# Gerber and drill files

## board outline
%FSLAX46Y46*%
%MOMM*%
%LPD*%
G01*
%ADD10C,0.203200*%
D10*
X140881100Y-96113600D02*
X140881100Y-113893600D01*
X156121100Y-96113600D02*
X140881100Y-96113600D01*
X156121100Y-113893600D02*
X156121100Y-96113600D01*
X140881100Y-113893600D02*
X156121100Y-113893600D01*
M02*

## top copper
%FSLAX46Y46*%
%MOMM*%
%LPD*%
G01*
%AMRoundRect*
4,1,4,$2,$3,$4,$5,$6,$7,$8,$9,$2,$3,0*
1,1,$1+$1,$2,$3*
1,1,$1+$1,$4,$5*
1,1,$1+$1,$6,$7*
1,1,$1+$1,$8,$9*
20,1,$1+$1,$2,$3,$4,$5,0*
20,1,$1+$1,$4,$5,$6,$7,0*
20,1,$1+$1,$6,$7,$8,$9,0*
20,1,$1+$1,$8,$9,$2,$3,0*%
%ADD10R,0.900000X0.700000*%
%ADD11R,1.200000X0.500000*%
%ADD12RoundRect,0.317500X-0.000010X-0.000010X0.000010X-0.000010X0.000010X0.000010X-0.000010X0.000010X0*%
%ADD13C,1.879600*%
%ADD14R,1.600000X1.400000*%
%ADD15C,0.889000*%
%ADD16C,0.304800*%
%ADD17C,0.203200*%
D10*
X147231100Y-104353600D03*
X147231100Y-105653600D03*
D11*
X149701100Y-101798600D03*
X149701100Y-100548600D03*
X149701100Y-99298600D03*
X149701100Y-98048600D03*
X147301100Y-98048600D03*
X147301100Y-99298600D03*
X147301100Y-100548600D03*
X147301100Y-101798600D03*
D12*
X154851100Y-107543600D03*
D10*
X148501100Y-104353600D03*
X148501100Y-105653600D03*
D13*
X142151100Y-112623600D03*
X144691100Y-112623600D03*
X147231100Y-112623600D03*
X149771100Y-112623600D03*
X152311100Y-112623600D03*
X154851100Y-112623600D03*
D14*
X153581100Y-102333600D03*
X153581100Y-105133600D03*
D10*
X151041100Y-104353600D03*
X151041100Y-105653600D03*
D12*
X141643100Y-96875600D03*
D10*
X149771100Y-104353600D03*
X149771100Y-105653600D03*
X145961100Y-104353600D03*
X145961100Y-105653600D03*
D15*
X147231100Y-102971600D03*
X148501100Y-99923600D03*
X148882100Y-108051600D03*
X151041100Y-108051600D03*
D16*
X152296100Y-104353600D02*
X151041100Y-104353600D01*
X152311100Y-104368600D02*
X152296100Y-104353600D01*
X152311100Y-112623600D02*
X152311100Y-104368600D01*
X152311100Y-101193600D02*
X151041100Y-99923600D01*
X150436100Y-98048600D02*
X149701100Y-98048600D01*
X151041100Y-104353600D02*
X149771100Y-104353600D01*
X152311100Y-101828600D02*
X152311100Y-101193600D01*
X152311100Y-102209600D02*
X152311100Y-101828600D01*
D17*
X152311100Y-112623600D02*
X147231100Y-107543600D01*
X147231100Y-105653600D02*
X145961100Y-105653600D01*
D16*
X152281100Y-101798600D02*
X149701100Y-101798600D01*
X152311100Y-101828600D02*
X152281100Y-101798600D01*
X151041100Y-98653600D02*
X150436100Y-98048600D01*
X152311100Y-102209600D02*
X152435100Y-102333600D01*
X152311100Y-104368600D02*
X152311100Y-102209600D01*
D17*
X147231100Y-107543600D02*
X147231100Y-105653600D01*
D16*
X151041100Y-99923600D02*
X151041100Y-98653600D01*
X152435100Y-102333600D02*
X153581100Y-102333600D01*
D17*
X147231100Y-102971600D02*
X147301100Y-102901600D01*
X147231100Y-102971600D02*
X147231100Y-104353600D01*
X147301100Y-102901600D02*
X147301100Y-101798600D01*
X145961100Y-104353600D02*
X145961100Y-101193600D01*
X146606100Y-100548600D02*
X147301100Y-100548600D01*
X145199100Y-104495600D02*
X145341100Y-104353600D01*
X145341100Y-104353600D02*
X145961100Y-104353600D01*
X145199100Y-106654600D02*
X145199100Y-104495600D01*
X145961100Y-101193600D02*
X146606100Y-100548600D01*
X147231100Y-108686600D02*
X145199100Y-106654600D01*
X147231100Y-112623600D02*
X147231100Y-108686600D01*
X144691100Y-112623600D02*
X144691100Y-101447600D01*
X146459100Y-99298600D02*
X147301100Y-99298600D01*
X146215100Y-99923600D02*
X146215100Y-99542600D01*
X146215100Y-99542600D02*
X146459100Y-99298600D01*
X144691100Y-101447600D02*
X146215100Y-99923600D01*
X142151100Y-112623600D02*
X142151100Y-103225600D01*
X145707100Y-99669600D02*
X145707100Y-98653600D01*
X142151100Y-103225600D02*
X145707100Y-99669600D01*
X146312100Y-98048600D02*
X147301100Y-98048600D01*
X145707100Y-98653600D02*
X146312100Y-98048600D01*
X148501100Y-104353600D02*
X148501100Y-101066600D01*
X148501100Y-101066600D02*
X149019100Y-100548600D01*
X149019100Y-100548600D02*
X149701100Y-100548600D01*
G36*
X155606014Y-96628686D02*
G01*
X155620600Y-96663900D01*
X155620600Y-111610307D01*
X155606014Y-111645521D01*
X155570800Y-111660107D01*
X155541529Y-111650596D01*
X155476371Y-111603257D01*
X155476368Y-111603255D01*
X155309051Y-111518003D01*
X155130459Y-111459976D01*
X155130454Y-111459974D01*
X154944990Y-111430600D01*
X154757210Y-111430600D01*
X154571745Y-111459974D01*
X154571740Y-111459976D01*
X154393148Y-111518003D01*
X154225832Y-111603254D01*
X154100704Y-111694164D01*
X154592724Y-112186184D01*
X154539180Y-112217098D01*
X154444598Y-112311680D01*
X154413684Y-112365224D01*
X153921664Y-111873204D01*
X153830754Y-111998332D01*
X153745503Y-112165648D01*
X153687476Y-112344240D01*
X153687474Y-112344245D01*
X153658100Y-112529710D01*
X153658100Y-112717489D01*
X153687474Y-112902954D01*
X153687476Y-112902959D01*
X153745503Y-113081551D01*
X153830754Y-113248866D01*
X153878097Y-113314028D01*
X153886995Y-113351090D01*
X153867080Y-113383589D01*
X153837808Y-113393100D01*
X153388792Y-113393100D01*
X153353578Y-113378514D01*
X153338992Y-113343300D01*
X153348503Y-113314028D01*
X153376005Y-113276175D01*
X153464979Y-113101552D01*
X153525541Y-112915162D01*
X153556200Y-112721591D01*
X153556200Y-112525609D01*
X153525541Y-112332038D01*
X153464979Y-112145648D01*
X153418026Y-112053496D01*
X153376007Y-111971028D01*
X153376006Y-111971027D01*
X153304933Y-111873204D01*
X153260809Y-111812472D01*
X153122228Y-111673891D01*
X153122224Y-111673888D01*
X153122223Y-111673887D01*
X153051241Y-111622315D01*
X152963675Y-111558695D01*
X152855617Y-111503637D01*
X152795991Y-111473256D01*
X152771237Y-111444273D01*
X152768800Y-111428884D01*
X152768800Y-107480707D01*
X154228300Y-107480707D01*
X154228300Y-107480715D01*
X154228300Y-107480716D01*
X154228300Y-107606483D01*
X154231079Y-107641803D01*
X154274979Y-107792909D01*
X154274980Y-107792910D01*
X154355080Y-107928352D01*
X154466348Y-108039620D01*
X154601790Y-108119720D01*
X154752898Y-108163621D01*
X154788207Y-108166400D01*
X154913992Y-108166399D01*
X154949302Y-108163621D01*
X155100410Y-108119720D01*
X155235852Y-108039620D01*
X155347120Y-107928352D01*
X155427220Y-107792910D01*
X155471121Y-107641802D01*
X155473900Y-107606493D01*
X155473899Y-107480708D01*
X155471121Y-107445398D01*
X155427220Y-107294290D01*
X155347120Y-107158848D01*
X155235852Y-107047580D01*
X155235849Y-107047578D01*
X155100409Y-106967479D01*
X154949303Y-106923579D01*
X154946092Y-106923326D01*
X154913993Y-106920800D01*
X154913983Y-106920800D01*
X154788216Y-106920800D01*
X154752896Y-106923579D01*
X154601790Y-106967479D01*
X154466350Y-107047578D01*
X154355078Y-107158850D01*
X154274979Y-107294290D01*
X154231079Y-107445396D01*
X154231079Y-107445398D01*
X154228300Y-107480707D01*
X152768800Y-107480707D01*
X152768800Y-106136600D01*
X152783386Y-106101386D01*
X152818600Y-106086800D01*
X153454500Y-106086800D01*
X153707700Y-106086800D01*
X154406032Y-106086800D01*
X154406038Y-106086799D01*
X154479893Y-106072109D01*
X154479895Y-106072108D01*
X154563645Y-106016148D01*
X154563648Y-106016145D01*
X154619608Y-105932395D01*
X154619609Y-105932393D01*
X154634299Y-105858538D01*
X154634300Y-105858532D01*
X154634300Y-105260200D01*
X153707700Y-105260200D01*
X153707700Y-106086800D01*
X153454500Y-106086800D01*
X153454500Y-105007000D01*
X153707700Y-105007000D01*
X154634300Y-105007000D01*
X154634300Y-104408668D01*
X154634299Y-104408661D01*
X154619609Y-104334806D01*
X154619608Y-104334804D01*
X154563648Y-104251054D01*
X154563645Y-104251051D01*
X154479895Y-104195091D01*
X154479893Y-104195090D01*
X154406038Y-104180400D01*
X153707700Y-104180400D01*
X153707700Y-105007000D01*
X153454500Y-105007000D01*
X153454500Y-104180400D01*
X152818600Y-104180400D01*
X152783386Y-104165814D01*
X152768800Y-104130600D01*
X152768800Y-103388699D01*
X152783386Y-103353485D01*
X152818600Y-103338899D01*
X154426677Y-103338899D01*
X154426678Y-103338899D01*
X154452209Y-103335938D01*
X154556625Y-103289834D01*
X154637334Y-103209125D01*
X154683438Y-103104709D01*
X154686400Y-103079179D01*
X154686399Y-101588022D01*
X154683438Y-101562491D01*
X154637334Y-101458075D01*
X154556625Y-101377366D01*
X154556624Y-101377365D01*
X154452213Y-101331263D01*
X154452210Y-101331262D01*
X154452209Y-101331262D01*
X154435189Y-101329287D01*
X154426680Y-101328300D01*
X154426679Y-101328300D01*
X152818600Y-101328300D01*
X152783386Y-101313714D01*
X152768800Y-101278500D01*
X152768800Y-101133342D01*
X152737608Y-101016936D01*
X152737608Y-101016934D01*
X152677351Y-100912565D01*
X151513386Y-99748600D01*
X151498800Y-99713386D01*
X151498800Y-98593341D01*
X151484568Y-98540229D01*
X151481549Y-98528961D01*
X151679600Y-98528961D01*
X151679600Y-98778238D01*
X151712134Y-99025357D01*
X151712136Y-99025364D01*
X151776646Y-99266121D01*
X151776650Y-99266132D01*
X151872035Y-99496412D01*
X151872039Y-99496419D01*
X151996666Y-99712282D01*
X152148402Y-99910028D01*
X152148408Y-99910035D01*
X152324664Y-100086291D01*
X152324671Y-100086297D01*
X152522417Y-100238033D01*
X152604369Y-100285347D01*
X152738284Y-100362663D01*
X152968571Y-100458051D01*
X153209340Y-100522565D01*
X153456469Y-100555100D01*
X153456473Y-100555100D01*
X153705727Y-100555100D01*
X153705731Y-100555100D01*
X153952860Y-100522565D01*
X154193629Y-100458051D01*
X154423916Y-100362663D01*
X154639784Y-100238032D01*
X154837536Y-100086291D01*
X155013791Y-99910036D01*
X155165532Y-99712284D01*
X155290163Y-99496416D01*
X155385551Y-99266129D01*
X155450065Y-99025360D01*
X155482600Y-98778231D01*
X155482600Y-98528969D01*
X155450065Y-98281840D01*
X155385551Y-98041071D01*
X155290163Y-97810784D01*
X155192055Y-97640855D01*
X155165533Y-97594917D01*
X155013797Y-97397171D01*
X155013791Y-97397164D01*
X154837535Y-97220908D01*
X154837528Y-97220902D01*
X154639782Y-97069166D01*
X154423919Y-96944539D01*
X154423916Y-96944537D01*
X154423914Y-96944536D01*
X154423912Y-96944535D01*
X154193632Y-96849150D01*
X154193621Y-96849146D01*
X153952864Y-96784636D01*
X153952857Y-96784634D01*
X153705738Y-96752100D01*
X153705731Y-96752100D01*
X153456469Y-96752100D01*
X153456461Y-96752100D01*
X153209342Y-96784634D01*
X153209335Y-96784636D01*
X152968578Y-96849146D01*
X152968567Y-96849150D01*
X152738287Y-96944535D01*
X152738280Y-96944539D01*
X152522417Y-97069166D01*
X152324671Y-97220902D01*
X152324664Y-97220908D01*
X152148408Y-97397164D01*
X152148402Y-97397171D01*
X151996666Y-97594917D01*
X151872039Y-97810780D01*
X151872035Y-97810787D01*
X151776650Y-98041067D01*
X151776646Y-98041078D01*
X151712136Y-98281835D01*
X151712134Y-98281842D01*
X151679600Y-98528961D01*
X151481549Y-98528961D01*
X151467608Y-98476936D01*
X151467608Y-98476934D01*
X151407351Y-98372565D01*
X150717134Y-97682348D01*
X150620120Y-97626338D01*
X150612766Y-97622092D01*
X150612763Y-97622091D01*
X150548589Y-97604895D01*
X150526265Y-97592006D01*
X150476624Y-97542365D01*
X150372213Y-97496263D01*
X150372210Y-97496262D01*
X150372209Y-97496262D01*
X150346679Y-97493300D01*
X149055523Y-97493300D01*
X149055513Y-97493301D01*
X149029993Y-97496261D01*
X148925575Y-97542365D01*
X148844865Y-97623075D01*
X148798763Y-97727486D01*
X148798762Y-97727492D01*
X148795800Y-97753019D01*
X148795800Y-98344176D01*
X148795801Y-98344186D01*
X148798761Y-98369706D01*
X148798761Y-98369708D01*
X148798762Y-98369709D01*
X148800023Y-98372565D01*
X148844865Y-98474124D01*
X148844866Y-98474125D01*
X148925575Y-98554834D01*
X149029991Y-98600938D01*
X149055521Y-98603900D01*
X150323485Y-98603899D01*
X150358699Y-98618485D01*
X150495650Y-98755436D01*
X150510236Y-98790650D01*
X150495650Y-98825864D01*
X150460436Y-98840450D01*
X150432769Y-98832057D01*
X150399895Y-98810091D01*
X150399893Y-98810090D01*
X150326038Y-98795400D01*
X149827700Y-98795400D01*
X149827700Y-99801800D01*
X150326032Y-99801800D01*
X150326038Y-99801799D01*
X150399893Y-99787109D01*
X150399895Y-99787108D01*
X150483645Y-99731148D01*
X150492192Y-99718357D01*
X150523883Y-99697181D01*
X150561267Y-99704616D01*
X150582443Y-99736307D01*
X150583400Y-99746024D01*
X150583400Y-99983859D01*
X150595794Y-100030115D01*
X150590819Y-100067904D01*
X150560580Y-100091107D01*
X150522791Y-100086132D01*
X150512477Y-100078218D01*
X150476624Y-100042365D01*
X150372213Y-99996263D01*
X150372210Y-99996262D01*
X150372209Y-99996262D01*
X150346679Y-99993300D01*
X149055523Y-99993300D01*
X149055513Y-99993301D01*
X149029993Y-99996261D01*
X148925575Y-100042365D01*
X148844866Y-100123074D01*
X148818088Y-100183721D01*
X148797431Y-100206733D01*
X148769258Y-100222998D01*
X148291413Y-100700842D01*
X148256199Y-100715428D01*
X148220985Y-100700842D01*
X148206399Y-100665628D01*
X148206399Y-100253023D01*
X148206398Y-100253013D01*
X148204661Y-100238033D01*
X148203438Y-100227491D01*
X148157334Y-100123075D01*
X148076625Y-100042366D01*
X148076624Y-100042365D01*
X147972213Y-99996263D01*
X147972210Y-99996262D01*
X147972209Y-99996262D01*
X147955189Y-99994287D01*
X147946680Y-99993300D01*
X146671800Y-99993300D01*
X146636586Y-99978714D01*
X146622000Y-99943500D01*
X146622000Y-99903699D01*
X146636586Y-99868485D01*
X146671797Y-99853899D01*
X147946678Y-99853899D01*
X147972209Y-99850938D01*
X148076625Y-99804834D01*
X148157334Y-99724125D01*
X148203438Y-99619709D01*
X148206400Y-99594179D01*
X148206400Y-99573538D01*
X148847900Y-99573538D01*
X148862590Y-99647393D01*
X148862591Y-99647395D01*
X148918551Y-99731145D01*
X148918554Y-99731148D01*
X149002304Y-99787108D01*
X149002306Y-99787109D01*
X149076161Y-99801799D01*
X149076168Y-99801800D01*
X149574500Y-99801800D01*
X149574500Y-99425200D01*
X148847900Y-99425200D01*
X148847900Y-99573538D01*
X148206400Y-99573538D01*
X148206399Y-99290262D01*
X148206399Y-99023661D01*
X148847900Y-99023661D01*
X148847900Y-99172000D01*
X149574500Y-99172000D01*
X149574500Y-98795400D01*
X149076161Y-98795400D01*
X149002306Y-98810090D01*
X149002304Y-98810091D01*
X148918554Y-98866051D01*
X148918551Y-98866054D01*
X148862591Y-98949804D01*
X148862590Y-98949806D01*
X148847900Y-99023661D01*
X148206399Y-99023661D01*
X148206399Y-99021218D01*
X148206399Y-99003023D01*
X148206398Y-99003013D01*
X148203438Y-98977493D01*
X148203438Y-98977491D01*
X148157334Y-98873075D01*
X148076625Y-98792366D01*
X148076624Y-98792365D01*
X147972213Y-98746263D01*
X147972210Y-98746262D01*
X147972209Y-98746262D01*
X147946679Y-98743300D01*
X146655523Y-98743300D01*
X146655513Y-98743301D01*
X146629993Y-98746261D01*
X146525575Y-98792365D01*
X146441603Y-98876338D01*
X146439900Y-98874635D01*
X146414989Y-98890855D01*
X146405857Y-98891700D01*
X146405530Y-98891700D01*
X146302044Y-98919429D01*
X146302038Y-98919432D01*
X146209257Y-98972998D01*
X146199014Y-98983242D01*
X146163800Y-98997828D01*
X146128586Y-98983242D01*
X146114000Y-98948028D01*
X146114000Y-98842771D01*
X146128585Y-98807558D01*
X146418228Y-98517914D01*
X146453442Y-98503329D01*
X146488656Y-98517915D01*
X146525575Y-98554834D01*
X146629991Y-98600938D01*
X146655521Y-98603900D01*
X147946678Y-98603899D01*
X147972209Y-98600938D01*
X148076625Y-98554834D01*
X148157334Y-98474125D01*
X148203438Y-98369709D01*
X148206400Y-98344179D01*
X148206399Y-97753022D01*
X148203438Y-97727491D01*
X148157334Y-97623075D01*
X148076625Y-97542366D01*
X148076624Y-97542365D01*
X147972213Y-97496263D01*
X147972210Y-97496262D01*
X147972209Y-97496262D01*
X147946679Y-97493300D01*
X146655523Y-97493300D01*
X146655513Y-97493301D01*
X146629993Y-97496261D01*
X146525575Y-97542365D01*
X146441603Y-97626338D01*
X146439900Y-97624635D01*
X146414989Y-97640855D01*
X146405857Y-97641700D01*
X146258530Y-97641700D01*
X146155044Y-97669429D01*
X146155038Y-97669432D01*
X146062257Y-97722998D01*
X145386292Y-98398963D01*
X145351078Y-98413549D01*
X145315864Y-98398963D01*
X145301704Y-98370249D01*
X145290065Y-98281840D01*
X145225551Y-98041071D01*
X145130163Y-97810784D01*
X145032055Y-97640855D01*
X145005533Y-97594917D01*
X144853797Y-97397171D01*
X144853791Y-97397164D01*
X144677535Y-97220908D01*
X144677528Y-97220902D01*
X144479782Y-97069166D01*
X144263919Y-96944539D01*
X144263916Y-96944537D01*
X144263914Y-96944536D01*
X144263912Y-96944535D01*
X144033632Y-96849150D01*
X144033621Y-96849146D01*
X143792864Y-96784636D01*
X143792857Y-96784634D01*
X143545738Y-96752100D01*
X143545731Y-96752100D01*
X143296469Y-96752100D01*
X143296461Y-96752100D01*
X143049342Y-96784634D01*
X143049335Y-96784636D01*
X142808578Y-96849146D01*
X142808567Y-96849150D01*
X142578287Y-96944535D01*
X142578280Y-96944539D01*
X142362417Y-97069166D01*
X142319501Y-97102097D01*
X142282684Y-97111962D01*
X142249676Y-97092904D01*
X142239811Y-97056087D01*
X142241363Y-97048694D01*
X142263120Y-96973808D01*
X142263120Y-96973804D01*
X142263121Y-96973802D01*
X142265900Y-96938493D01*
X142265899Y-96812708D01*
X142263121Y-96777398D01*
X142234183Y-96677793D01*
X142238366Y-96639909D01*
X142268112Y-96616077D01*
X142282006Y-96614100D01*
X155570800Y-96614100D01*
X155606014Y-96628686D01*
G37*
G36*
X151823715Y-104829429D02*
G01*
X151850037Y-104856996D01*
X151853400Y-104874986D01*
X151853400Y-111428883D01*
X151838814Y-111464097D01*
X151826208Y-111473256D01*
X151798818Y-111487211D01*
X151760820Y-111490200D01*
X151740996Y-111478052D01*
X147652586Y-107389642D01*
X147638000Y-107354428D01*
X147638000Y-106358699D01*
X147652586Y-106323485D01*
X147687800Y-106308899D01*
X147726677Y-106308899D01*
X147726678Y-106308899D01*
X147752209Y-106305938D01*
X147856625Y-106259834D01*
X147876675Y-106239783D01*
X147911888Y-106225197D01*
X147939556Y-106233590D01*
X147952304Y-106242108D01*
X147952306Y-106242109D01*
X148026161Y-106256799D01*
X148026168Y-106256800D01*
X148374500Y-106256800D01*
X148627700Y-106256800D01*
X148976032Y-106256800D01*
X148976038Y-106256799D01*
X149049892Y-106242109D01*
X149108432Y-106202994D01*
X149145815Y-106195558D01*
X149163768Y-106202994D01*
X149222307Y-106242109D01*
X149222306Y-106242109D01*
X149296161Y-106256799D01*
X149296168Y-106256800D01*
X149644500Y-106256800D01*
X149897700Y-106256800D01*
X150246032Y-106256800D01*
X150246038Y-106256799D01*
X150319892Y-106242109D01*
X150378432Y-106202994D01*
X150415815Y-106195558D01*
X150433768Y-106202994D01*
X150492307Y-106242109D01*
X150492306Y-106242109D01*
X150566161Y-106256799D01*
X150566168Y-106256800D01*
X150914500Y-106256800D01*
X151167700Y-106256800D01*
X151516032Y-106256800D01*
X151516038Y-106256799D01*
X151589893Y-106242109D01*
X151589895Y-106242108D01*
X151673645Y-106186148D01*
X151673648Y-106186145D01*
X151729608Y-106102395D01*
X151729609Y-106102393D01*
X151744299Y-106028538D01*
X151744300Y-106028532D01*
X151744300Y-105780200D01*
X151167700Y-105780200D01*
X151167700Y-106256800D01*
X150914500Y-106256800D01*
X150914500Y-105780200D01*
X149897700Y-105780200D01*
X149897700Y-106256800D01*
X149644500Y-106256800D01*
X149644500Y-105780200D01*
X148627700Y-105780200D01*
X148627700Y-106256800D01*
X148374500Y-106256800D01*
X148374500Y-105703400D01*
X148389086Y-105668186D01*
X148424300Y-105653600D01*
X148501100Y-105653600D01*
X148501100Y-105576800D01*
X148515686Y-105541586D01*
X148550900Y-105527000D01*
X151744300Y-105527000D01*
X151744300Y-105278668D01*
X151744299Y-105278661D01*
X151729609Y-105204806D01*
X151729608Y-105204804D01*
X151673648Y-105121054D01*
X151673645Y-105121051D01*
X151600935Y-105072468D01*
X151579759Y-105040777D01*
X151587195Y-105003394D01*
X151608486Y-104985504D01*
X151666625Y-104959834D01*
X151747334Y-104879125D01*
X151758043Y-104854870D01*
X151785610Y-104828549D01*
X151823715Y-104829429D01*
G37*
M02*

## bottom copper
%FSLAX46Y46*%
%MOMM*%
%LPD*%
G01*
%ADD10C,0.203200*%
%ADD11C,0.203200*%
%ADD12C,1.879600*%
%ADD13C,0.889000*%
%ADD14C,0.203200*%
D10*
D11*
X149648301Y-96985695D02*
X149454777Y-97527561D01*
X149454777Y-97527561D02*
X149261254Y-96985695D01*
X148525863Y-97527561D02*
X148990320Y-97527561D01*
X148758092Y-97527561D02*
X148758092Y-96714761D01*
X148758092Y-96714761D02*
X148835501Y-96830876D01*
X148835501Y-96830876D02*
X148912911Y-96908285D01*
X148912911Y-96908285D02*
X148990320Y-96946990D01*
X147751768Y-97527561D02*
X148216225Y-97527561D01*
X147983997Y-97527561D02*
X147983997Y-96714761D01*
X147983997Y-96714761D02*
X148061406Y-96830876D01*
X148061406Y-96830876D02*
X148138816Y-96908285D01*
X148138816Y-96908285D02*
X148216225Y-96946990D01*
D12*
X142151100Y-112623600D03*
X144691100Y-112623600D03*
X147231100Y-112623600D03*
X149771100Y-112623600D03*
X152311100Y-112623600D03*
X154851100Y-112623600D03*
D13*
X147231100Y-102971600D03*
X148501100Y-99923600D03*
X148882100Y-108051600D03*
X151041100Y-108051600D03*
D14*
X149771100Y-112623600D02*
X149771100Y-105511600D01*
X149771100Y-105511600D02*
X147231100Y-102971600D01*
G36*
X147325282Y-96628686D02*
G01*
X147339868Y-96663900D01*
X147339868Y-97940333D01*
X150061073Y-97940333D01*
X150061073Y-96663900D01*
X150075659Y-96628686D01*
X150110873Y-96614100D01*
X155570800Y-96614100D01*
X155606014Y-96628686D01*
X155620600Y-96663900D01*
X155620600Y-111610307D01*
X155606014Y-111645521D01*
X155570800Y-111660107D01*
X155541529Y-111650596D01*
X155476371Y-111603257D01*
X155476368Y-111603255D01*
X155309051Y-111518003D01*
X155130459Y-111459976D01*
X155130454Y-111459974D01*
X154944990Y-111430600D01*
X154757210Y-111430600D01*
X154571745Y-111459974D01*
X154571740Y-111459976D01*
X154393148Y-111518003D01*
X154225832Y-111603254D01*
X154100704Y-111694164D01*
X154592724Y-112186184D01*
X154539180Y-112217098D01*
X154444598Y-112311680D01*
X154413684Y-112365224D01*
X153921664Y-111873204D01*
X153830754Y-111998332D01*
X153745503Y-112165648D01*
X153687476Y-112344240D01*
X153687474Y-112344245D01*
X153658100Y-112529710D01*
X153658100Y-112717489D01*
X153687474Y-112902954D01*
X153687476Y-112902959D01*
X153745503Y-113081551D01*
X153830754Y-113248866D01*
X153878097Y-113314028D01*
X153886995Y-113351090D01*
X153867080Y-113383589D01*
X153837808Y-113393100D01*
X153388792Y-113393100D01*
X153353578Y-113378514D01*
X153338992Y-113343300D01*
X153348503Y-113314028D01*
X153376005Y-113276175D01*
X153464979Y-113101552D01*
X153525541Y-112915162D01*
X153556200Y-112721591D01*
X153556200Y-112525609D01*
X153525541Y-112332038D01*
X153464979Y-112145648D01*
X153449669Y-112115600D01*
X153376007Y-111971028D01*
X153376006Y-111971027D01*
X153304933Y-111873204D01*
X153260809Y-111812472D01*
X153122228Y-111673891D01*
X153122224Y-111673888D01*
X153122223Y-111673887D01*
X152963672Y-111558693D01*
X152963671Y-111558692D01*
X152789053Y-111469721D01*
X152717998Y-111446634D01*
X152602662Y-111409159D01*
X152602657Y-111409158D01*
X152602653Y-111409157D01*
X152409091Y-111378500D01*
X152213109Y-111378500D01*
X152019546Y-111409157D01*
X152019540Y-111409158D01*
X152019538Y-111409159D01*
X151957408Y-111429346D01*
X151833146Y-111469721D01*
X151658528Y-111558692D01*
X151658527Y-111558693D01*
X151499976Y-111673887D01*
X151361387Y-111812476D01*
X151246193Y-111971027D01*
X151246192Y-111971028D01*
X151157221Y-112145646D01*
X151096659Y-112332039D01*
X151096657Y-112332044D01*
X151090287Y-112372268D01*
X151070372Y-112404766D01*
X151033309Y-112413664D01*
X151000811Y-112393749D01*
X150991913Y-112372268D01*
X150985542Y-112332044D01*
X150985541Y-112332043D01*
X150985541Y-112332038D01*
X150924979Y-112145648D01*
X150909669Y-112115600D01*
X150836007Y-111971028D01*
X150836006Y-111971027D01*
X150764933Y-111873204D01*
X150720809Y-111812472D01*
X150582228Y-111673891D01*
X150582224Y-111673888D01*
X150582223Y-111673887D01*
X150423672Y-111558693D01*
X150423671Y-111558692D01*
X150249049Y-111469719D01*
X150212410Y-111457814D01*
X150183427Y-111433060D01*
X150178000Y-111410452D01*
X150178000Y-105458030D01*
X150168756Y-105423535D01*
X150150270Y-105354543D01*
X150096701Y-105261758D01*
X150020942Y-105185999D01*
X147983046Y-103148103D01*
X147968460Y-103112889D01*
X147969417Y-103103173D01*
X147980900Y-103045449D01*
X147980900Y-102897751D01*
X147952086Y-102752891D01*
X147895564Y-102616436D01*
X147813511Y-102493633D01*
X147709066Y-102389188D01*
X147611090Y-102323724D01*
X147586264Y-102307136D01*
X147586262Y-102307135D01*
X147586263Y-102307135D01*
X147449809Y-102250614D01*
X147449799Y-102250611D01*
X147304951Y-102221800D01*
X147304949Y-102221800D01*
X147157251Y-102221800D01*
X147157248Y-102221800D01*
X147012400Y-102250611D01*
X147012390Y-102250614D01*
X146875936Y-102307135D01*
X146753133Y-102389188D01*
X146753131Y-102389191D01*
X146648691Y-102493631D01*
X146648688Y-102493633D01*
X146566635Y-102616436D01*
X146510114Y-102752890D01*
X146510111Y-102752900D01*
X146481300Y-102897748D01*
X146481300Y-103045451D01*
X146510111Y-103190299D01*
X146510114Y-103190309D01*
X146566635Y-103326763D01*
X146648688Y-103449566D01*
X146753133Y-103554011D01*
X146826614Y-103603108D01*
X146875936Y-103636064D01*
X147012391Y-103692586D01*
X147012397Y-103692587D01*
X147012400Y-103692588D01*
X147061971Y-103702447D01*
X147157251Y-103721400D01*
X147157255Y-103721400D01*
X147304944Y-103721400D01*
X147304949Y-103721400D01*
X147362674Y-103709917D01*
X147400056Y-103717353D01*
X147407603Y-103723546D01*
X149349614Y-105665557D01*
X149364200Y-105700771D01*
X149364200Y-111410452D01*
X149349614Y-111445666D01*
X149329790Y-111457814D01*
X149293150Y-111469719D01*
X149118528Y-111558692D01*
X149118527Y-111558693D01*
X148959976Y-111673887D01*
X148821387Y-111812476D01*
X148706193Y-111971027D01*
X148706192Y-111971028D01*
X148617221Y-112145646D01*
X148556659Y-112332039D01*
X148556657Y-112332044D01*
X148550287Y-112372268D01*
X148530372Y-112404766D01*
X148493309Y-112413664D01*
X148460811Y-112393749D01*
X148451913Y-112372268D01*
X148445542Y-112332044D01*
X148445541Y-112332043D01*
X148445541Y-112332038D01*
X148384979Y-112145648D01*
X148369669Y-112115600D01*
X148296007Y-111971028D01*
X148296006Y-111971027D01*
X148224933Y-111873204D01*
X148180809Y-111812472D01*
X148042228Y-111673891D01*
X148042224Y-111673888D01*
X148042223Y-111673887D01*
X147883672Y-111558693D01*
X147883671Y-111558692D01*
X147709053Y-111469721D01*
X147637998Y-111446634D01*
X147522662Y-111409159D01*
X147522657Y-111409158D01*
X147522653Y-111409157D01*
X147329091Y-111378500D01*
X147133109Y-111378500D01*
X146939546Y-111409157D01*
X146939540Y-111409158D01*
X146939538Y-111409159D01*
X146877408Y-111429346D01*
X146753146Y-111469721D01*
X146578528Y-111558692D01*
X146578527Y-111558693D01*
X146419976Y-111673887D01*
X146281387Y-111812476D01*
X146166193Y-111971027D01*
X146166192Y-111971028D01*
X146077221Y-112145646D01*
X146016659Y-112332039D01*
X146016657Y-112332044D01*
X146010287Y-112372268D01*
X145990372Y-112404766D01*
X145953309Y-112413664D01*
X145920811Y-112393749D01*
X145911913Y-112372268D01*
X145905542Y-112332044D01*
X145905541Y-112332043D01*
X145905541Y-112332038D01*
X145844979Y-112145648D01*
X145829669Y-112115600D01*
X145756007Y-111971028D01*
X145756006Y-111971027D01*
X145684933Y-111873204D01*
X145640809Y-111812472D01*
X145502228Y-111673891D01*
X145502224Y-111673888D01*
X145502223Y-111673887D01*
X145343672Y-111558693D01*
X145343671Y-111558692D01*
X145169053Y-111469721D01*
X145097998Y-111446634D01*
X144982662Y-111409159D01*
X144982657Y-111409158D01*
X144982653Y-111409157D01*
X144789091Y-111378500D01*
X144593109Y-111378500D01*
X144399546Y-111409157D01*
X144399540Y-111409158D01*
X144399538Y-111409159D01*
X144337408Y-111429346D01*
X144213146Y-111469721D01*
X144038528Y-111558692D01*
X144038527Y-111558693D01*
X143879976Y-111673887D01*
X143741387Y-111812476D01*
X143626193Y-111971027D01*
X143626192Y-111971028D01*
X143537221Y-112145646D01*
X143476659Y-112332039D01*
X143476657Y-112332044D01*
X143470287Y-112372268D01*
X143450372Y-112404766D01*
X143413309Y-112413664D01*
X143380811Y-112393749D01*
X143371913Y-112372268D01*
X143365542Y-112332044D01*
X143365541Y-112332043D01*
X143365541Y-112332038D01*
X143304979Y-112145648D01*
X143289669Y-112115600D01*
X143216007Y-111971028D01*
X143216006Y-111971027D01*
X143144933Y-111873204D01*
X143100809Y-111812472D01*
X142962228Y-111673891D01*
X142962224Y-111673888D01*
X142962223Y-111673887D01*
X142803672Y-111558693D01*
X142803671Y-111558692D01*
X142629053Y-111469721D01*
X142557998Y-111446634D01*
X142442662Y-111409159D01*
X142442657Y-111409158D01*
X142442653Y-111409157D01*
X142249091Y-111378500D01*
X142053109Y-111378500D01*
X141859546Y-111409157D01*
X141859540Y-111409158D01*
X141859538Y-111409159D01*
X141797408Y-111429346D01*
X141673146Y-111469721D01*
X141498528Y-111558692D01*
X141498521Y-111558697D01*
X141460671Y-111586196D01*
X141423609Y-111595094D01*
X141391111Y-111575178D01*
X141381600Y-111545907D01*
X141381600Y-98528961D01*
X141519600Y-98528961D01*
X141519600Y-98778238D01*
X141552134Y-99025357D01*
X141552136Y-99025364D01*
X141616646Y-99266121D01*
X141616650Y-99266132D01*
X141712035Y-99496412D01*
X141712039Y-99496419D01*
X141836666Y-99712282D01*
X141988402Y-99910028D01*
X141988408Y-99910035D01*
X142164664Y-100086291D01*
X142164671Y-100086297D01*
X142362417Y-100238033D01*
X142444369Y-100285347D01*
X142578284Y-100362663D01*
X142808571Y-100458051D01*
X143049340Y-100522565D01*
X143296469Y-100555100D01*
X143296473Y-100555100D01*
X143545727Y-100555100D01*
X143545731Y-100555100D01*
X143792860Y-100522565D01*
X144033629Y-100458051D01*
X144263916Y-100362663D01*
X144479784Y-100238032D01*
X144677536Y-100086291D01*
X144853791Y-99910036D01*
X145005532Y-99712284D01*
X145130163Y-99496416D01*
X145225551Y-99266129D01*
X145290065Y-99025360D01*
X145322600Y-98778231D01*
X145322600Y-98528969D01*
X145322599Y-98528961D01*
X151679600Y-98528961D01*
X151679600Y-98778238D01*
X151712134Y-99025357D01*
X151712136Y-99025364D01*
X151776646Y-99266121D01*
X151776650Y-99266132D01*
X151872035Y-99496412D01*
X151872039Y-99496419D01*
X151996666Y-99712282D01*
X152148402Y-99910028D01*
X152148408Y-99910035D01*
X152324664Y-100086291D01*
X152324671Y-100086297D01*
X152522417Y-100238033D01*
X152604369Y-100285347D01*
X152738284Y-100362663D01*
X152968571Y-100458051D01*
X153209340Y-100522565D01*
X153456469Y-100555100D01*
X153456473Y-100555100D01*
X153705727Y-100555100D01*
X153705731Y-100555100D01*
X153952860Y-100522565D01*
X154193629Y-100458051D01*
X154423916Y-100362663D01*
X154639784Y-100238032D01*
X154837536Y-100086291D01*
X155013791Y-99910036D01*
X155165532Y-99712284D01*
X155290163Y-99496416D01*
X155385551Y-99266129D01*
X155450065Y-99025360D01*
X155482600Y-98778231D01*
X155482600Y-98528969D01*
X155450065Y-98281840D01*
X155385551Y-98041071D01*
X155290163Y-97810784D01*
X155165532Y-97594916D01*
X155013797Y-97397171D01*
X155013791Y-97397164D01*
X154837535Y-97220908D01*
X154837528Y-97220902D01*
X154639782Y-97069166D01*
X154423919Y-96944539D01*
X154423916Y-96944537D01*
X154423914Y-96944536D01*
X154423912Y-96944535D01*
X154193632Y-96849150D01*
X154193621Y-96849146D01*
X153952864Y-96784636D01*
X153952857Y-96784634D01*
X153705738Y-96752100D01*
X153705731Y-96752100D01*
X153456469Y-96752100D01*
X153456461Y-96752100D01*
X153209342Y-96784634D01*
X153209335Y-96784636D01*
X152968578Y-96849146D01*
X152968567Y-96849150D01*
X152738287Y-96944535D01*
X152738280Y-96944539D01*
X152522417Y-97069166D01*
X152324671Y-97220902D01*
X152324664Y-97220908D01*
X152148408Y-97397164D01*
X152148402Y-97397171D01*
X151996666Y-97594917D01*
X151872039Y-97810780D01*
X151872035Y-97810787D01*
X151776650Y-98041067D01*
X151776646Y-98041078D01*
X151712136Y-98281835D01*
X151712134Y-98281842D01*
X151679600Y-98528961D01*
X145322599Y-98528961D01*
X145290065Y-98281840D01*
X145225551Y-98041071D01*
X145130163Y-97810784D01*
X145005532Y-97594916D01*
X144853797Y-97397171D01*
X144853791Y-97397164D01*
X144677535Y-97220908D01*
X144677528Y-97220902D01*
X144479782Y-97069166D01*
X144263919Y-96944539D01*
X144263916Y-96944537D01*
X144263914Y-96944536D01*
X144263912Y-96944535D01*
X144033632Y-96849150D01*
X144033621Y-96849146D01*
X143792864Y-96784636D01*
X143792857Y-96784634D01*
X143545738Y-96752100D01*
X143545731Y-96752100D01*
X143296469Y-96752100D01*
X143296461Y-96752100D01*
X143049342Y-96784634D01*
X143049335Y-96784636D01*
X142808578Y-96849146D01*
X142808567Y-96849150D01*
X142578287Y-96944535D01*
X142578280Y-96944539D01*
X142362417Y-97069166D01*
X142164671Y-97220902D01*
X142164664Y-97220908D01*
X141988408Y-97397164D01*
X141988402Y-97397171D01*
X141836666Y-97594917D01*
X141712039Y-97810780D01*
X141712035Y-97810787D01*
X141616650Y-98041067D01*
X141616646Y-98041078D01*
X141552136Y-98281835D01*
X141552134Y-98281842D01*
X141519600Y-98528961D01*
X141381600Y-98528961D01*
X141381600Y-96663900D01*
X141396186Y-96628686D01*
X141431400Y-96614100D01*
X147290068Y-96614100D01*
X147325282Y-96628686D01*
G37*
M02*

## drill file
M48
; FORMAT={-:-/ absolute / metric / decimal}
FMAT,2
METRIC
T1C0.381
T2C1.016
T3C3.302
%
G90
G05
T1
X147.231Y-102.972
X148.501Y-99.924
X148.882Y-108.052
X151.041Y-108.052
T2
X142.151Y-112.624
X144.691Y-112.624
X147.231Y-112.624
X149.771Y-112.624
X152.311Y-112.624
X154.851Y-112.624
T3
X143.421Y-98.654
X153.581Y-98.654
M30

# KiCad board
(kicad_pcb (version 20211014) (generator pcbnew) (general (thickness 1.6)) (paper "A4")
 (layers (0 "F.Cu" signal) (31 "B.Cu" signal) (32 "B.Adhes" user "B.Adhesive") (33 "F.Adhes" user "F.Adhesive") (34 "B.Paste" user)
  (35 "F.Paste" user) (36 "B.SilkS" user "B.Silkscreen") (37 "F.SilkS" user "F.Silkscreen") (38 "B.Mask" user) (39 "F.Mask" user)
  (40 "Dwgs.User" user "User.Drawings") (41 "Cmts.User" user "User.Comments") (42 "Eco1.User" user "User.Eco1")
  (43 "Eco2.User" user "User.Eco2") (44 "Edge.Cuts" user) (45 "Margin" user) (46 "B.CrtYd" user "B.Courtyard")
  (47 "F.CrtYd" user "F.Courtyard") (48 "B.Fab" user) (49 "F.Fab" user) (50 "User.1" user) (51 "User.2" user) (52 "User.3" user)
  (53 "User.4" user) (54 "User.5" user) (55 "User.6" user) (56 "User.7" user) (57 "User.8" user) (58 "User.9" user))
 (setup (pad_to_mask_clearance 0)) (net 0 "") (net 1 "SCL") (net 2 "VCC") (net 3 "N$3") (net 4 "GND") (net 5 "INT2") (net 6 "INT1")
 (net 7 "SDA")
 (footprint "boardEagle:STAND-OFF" (layer "F.Cu") (at 143.4211 98.6536 180)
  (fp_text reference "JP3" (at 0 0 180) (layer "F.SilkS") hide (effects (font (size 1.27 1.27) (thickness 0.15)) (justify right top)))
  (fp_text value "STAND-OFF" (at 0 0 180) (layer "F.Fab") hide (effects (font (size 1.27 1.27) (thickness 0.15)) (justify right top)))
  (pad "" np_thru_hole circle (at 0 0 180) (size 3.302 3.302) (drill 3.302) (layers *.Cu *.Mask)))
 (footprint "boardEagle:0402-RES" (layer "F.Cu") (at 147.2311 105.0036 -90)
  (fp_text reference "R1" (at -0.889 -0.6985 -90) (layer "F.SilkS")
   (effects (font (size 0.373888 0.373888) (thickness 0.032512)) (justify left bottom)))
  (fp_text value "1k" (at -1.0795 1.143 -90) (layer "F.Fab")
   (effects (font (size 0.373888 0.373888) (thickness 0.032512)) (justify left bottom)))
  (pad "1" smd rect (at -0.65 0 270) (size 0.7 0.9) (layers "F.Cu" "F.Paste" "F.Mask") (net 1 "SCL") (solder_mask_margin 0.1016))
  (pad "2" smd rect (at 0.65 0 270) (size 0.7 0.9) (layers "F.Cu" "F.Paste" "F.Mask") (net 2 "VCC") (solder_mask_margin 0.1016)))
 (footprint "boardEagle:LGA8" (layer "F.Cu") (at 148.5011 99.9236 180)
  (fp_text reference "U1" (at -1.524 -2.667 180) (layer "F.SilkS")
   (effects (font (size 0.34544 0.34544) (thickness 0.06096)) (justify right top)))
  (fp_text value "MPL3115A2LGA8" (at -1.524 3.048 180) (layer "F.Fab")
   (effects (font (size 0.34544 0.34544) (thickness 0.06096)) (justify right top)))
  (pad "1" smd rect (at -1.2 -1.875 180) (size 1.2 0.5) (layers "F.Cu" "F.Paste" "F.Mask") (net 2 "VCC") (solder_mask_margin 0.1016))
  (pad "2" smd rect (at -1.2 -0.625 180) (size 1.2 0.5) (layers "F.Cu" "F.Paste" "F.Mask") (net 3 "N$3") (solder_mask_margin 0.1016))
  (pad "3" smd rect (at -1.2 0.625 180) (size 1.2 0.5) (layers "F.Cu" "F.Paste" "F.Mask") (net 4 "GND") (solder_mask_margin 0.1016))
  (pad "4" smd rect (at -1.2 1.875 180) (size 1.2 0.5) (layers "F.Cu" "F.Paste" "F.Mask") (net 2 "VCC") (solder_mask_margin 0.1016))
  (pad "5" smd rect (at 1.2 1.875 180) (size 1.2 0.5) (layers "F.Cu" "F.Paste" "F.Mask") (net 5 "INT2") (solder_mask_margin 0.1016))
  (pad "6" smd rect (at 1.2 0.625 180) (size 1.2 0.5) (layers "F.Cu" "F.Paste" "F.Mask") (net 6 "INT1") (solder_mask_margin 0.1016))
  (pad "7" smd rect (at 1.2 -0.625 180) (size 1.2 0.5) (layers "F.Cu" "F.Paste" "F.Mask") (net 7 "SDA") (solder_mask_margin 0.1016))
  (pad "8" smd rect (at 1.2 -1.875 180) (size 1.2 0.5) (layers "F.Cu" "F.Paste" "F.Mask") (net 1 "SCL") (solder_mask_margin 0.1016)))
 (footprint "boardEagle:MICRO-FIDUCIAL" (layer "F.Cu") (at 154.8511 107.5436)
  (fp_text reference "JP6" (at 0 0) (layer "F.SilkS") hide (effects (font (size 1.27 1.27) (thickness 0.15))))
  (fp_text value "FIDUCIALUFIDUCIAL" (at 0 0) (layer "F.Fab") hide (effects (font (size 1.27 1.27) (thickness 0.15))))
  (pad "1" smd roundrect (at 0 0) (size 0.635 0.635) (layers "F.Cu" "F.Mask") (roundrect_rratio 0.5) (solder_mask_margin 0.1016)))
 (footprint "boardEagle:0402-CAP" (layer "F.Cu") (at 148.5011 105.0036 -90)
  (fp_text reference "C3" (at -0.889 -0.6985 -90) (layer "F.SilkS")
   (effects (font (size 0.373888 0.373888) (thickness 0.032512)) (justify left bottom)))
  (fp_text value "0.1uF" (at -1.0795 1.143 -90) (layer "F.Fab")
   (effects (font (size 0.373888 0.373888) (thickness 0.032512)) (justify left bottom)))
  (pad "1" smd rect (at -0.65 0 270) (size 0.7 0.9) (layers "F.Cu" "F.Paste" "F.Mask") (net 3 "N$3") (solder_mask_margin 0.1016))
  (pad "2" smd rect (at 0.65 0 270) (size 0.7 0.9) (layers "F.Cu" "F.Paste" "F.Mask") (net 4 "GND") (solder_mask_margin 0.1016)))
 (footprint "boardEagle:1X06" (layer "F.Cu") (at 142.1511 112.6236)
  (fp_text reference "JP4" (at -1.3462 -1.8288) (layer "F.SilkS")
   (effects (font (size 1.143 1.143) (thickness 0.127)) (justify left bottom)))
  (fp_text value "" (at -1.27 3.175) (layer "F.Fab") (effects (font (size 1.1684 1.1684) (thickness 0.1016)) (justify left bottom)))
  (pad "1" thru_hole circle (at 0 0 90) (size 1.8796 1.8796) (drill 1.016) (layers *.Cu *.Mask) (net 5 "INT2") (solder_mask_margin 0.1016))
  (pad "2" thru_hole circle (at 2.54 0 90) (size 1.8796 1.8796) (drill 1.016) (layers *.Cu *.Mask) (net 6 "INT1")
   (solder_mask_margin 0.1016))
  (pad "3" thru_hole circle (at 5.08 0 90) (size 1.8796 1.8796) (drill 1.016) (layers *.Cu *.Mask) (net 7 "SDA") (solder_mask_margin 0.1016))
  (pad "4" thru_hole circle (at 7.62 0 90) (size 1.8796 1.8796) (drill 1.016) (layers *.Cu *.Mask) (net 1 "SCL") (solder_mask_margin 0.1016))
  (pad "5" thru_hole circle (at 10.16 0 90) (size 1.8796 1.8796) (drill 1.016) (layers *.Cu *.Mask) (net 2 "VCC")
   (solder_mask_margin 0.1016))
  (pad "6" thru_hole circle (at 12.7 0 90) (size 1.8796 1.8796) (drill 1.016) (layers *.Cu *.Mask) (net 4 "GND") (solder_mask_margin 0.1016)))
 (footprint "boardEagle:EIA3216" (layer "F.Cu") (at 153.5811 103.7336 90)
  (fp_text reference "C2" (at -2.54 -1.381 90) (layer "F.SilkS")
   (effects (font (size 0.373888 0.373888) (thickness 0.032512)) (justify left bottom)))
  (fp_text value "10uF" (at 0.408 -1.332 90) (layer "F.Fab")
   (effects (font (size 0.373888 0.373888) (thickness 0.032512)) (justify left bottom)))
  (pad "A" smd rect (at 1.4 0 180) (size 1.6 1.4) (layers "F.Cu" "F.Paste" "F.Mask") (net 2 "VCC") (solder_mask_margin 0.1016))
  (pad "C" smd rect (at -1.4 0 180) (size 1.6 1.4) (layers "F.Cu" "F.Paste" "F.Mask") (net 4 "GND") (solder_mask_margin 0.1016)))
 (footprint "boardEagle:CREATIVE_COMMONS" (layer "F.Cu") (at 157.3911 124.0536)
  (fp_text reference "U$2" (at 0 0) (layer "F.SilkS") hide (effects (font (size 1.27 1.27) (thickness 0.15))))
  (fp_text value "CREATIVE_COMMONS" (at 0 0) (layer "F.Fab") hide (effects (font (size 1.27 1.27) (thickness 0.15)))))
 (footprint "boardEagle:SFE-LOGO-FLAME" (layer "F.Cu") (at 142.7861 104.3686)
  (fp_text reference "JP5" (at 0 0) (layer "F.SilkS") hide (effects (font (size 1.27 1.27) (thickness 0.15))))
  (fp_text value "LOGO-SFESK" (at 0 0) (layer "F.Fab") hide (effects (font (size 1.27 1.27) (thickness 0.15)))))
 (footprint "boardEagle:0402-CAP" (layer "F.Cu") (at 151.0411 105.0036 -90)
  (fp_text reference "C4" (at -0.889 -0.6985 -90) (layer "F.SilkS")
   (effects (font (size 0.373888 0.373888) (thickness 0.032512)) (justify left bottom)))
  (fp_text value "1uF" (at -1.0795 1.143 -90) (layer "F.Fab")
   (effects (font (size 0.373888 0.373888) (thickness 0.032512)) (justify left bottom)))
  (pad "1" smd rect (at -0.65 0 270) (size 0.7 0.9) (layers "F.Cu" "F.Paste" "F.Mask") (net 2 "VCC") (solder_mask_margin 0.1016))
  (pad "2" smd rect (at 0.65 0 270) (size 0.7 0.9) (layers "F.Cu" "F.Paste" "F.Mask") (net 4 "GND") (solder_mask_margin 0.1016)))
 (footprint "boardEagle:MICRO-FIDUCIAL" (layer "F.Cu") (at 141.6431 96.8756)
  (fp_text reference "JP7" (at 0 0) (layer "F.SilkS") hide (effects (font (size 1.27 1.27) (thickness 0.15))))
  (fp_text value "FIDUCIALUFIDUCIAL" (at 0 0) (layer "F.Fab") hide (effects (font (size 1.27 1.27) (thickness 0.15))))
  (pad "1" smd roundrect (at 0 0) (size 0.635 0.635) (layers "F.Cu" "F.Mask") (roundrect_rratio 0.5) (solder_mask_margin 0.1016)))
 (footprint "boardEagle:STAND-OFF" (layer "F.Cu") (at 153.5811 98.6536 180)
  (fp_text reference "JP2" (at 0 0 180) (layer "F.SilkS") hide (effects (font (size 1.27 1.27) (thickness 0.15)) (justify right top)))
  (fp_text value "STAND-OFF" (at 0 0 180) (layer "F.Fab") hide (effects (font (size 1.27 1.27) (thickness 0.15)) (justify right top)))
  (pad "" np_thru_hole circle (at 0 0 180) (size 3.302 3.302) (drill 3.302) (layers *.Cu *.Mask)))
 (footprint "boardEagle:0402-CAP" (layer "F.Cu") (at 149.7711 105.0036 -90)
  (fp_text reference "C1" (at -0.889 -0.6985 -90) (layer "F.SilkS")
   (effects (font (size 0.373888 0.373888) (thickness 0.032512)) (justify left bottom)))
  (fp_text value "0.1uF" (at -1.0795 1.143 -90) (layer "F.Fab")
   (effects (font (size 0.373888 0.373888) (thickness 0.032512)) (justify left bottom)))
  (pad "1" smd rect (at -0.65 0 270) (size 0.7 0.9) (layers "F.Cu" "F.Paste" "F.Mask") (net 2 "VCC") (solder_mask_margin 0.1016))
  (pad "2" smd rect (at 0.65 0 270) (size 0.7 0.9) (layers "F.Cu" "F.Paste" "F.Mask") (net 4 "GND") (solder_mask_margin 0.1016)))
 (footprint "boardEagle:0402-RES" (layer "F.Cu") (at 145.9611 105.0036 -90)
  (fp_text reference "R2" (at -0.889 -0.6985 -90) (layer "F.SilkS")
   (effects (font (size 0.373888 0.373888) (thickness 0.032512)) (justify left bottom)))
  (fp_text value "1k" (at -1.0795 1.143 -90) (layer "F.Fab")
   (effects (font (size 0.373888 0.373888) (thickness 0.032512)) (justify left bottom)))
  (pad "1" smd rect (at -0.65 0 270) (size 0.7 0.9) (layers "F.Cu" "F.Paste" "F.Mask") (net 7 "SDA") (solder_mask_margin 0.1016))
  (pad "2" smd rect (at 0.65 0 270) (size 0.7 0.9) (layers "F.Cu" "F.Paste" "F.Mask") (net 2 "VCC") (solder_mask_margin 0.1016)))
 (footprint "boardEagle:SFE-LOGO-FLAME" (layer "B.Cu") (at 144.0561 110.5916 180)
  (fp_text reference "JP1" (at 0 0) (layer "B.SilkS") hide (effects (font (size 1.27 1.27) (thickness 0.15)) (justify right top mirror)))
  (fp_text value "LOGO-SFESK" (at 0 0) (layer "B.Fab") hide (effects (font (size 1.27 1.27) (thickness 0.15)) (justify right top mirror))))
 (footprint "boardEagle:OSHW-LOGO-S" (layer "B.Cu") (at 153.5811 109.7026 180)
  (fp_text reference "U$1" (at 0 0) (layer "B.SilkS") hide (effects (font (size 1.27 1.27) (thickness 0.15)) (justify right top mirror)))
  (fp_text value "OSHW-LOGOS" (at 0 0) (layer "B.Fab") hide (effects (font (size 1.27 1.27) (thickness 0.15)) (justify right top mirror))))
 (gr_line (start 140.8811 96.1136) (end 140.8811 113.8936) (layer "Edge.Cuts") (width 0.2032))
 (gr_line (start 156.1211 96.1136) (end 140.8811 96.1136) (layer "Edge.Cuts") (width 0.2032))
 (gr_line (start 156.1211 113.8936) (end 156.1211 96.1136) (layer "Edge.Cuts") (width 0.2032))
 (gr_line (start 140.8811 113.8936) (end 156.1211 113.8936) (layer "Edge.Cuts") (width 0.2032))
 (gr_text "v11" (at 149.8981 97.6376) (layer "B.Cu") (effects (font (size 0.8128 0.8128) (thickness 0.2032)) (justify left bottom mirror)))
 (segment (start 152.2961 104.3536) (end 151.0411 104.3536) (width 0.3048) (layer "F.Cu") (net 2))
 (segment (start 152.3111 104.3686) (end 152.2961 104.3536) (width 0.3048) (layer "F.Cu") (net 2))
 (segment (start 152.3111 112.6236) (end 152.3111 104.3686) (width 0.3048) (layer "F.Cu") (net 2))
 (segment (start 152.3111 101.1936) (end 151.0411 99.9236) (width 0.3048) (layer "F.Cu") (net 2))
 (segment (start 150.4361 98.0486) (end 149.7011 98.0486) (width 0.3048) (layer "F.Cu") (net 2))
 (segment (start 151.0411 104.3536) (end 149.7711 104.3536) (width 0.3048) (layer "F.Cu") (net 2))
 (segment (start 152.3111 101.8286) (end 152.3111 101.1936) (width 0.3048) (layer "F.Cu") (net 2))
 (segment (start 152.3111 102.2096) (end 152.3111 101.8286) (width 0.3048) (layer "F.Cu") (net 2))
 (segment (start 152.3111 112.6236) (end 147.2311 107.5436) (width 0.2032) (layer "F.Cu") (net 2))
 (segment (start 147.2311 105.6536) (end 145.9611 105.6536) (width 0.2032) (layer "F.Cu") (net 2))
 (segment (start 152.2811 101.7986) (end 149.7011 101.7986) (width 0.3048) (layer "F.Cu") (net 2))
 (segment (start 152.3111 101.8286) (end 152.2811 101.7986) (width 0.3048) (layer "F.Cu") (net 2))
 (segment (start 151.0411 98.6536) (end 150.4361 98.0486) (width 0.3048) (layer "F.Cu") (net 2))
 (segment (start 152.3111 102.2096) (end 152.4351 102.3336) (width 0.3048) (layer "F.Cu") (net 2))
 (segment (start 152.3111 104.3686) (end 152.3111 102.2096) (width 0.3048) (layer "F.Cu") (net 2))
 (segment (start 147.2311 107.5436) (end 147.2311 105.6536) (width 0.2032) (layer "F.Cu") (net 2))
 (segment (start 151.0411 99.9236) (end 151.0411 98.6536) (width 0.3048) (layer "F.Cu") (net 2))
 (segment (start 152.4351 102.3336) (end 153.5811 102.3336) (width 0.3048) (layer "F.Cu") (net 2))
 (segment (start 147.2311 102.9716) (end 147.3011 102.9016) (width 0.2032) (layer "F.Cu") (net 1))
 (segment (start 147.2311 102.9716) (end 147.2311 104.3536) (width 0.2032) (layer "F.Cu") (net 1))
 (segment (start 147.3011 102.9016) (end 147.3011 101.7986) (width 0.2032) (layer "F.Cu") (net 1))
 (via (at 147.2311 102.9716) (size 0.889) (drill 0.381) (layers "F.Cu" "B.Cu") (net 1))
 (segment (start 149.7711 112.6236) (end 149.7711 105.5116) (width 0.2032) (layer "B.Cu") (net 1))
 (segment (start 149.7711 105.5116) (end 147.2311 102.9716) (width 0.2032) (layer "B.Cu") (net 1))
 (segment (start 145.9611 104.3536) (end 145.9611 101.1936) (width 0.2032) (layer "F.Cu") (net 7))
 (segment (start 146.6061 100.5486) (end 147.3011 100.5486) (width 0.2032) (layer "F.Cu") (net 7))
 (segment (start 145.1991 104.4956) (end 145.3411 104.3536) (width 0.2032) (layer "F.Cu") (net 7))
 (segment (start 145.3411 104.3536) (end 145.9611 104.3536) (width 0.2032) (layer "F.Cu") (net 7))
 (segment (start 145.1991 106.6546) (end 145.1991 104.4956) (width 0.2032) (layer "F.Cu") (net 7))
 (segment (start 145.9611 101.1936) (end 146.6061 100.5486) (width 0.2032) (layer "F.Cu") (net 7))
 (segment (start 147.2311 108.6866) (end 145.1991 106.6546) (width 0.2032) (layer "F.Cu") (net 7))
 (segment (start 147.2311 112.6236) (end 147.2311 108.6866) (width 0.2032) (layer "F.Cu") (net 7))
 (segment (start 144.6911 112.6236) (end 144.6911 101.4476) (width 0.2032) (layer "F.Cu") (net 6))
 (segment (start 146.4591 99.2986) (end 147.3011 99.2986) (width 0.2032) (layer "F.Cu") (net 6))
 (segment (start 146.2151 99.9236) (end 146.2151 99.5426) (width 0.2032) (layer "F.Cu") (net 6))
 (segment (start 146.2151 99.5426) (end 146.4591 99.2986) (width 0.2032) (layer "F.Cu") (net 6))
 (segment (start 144.6911 101.4476) (end 146.2151 99.9236) (width 0.2032) (layer "F.Cu") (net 6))
 (segment (start 142.1511 112.6236) (end 142.1511 103.2256) (width 0.2032) (layer "F.Cu") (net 5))
 (segment (start 145.7071 99.6696) (end 145.7071 98.6536) (width 0.2032) (layer "F.Cu") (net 5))
 (segment (start 142.1511 103.2256) (end 145.7071 99.6696) (width 0.2032) (layer "F.Cu") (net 5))
 (segment (start 146.3121 98.0486) (end 147.3011 98.0486) (width 0.2032) (layer "F.Cu") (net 5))
 (segment (start 145.7071 98.6536) (end 146.3121 98.0486) (width 0.2032) (layer "F.Cu") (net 5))
 (segment (start 148.5011 104.3536) (end 148.5011 101.0666) (width 0.2032) (layer "F.Cu") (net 3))
 (segment (start 148.5011 101.0666) (end 149.0191 100.5486) (width 0.2032) (layer "F.Cu") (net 3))
 (segment (start 149.0191 100.5486) (end 149.7011 100.5486) (width 0.2032) (layer "F.Cu") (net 3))
 (via (at 148.5011 99.9236) (size 0.889) (drill 0.381) (layers "F.Cu" "B.Cu") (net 4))
 (via (at 148.8821 108.0516) (size 0.889) (drill 0.381) (layers "F.Cu" "B.Cu") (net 4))
 (via (at 151.0411 108.0516) (size 0.889) (drill 0.381) (layers "F.Cu" "B.Cu") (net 4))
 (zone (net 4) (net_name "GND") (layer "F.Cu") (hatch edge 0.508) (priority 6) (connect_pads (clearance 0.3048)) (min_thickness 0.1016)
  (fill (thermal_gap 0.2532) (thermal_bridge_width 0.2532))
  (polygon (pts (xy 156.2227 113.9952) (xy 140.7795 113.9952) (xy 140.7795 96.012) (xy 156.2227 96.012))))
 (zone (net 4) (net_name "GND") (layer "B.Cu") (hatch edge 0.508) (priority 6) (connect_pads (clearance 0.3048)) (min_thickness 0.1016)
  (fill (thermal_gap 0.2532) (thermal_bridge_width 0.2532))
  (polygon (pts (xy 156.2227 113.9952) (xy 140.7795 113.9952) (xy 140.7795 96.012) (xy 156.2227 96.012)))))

